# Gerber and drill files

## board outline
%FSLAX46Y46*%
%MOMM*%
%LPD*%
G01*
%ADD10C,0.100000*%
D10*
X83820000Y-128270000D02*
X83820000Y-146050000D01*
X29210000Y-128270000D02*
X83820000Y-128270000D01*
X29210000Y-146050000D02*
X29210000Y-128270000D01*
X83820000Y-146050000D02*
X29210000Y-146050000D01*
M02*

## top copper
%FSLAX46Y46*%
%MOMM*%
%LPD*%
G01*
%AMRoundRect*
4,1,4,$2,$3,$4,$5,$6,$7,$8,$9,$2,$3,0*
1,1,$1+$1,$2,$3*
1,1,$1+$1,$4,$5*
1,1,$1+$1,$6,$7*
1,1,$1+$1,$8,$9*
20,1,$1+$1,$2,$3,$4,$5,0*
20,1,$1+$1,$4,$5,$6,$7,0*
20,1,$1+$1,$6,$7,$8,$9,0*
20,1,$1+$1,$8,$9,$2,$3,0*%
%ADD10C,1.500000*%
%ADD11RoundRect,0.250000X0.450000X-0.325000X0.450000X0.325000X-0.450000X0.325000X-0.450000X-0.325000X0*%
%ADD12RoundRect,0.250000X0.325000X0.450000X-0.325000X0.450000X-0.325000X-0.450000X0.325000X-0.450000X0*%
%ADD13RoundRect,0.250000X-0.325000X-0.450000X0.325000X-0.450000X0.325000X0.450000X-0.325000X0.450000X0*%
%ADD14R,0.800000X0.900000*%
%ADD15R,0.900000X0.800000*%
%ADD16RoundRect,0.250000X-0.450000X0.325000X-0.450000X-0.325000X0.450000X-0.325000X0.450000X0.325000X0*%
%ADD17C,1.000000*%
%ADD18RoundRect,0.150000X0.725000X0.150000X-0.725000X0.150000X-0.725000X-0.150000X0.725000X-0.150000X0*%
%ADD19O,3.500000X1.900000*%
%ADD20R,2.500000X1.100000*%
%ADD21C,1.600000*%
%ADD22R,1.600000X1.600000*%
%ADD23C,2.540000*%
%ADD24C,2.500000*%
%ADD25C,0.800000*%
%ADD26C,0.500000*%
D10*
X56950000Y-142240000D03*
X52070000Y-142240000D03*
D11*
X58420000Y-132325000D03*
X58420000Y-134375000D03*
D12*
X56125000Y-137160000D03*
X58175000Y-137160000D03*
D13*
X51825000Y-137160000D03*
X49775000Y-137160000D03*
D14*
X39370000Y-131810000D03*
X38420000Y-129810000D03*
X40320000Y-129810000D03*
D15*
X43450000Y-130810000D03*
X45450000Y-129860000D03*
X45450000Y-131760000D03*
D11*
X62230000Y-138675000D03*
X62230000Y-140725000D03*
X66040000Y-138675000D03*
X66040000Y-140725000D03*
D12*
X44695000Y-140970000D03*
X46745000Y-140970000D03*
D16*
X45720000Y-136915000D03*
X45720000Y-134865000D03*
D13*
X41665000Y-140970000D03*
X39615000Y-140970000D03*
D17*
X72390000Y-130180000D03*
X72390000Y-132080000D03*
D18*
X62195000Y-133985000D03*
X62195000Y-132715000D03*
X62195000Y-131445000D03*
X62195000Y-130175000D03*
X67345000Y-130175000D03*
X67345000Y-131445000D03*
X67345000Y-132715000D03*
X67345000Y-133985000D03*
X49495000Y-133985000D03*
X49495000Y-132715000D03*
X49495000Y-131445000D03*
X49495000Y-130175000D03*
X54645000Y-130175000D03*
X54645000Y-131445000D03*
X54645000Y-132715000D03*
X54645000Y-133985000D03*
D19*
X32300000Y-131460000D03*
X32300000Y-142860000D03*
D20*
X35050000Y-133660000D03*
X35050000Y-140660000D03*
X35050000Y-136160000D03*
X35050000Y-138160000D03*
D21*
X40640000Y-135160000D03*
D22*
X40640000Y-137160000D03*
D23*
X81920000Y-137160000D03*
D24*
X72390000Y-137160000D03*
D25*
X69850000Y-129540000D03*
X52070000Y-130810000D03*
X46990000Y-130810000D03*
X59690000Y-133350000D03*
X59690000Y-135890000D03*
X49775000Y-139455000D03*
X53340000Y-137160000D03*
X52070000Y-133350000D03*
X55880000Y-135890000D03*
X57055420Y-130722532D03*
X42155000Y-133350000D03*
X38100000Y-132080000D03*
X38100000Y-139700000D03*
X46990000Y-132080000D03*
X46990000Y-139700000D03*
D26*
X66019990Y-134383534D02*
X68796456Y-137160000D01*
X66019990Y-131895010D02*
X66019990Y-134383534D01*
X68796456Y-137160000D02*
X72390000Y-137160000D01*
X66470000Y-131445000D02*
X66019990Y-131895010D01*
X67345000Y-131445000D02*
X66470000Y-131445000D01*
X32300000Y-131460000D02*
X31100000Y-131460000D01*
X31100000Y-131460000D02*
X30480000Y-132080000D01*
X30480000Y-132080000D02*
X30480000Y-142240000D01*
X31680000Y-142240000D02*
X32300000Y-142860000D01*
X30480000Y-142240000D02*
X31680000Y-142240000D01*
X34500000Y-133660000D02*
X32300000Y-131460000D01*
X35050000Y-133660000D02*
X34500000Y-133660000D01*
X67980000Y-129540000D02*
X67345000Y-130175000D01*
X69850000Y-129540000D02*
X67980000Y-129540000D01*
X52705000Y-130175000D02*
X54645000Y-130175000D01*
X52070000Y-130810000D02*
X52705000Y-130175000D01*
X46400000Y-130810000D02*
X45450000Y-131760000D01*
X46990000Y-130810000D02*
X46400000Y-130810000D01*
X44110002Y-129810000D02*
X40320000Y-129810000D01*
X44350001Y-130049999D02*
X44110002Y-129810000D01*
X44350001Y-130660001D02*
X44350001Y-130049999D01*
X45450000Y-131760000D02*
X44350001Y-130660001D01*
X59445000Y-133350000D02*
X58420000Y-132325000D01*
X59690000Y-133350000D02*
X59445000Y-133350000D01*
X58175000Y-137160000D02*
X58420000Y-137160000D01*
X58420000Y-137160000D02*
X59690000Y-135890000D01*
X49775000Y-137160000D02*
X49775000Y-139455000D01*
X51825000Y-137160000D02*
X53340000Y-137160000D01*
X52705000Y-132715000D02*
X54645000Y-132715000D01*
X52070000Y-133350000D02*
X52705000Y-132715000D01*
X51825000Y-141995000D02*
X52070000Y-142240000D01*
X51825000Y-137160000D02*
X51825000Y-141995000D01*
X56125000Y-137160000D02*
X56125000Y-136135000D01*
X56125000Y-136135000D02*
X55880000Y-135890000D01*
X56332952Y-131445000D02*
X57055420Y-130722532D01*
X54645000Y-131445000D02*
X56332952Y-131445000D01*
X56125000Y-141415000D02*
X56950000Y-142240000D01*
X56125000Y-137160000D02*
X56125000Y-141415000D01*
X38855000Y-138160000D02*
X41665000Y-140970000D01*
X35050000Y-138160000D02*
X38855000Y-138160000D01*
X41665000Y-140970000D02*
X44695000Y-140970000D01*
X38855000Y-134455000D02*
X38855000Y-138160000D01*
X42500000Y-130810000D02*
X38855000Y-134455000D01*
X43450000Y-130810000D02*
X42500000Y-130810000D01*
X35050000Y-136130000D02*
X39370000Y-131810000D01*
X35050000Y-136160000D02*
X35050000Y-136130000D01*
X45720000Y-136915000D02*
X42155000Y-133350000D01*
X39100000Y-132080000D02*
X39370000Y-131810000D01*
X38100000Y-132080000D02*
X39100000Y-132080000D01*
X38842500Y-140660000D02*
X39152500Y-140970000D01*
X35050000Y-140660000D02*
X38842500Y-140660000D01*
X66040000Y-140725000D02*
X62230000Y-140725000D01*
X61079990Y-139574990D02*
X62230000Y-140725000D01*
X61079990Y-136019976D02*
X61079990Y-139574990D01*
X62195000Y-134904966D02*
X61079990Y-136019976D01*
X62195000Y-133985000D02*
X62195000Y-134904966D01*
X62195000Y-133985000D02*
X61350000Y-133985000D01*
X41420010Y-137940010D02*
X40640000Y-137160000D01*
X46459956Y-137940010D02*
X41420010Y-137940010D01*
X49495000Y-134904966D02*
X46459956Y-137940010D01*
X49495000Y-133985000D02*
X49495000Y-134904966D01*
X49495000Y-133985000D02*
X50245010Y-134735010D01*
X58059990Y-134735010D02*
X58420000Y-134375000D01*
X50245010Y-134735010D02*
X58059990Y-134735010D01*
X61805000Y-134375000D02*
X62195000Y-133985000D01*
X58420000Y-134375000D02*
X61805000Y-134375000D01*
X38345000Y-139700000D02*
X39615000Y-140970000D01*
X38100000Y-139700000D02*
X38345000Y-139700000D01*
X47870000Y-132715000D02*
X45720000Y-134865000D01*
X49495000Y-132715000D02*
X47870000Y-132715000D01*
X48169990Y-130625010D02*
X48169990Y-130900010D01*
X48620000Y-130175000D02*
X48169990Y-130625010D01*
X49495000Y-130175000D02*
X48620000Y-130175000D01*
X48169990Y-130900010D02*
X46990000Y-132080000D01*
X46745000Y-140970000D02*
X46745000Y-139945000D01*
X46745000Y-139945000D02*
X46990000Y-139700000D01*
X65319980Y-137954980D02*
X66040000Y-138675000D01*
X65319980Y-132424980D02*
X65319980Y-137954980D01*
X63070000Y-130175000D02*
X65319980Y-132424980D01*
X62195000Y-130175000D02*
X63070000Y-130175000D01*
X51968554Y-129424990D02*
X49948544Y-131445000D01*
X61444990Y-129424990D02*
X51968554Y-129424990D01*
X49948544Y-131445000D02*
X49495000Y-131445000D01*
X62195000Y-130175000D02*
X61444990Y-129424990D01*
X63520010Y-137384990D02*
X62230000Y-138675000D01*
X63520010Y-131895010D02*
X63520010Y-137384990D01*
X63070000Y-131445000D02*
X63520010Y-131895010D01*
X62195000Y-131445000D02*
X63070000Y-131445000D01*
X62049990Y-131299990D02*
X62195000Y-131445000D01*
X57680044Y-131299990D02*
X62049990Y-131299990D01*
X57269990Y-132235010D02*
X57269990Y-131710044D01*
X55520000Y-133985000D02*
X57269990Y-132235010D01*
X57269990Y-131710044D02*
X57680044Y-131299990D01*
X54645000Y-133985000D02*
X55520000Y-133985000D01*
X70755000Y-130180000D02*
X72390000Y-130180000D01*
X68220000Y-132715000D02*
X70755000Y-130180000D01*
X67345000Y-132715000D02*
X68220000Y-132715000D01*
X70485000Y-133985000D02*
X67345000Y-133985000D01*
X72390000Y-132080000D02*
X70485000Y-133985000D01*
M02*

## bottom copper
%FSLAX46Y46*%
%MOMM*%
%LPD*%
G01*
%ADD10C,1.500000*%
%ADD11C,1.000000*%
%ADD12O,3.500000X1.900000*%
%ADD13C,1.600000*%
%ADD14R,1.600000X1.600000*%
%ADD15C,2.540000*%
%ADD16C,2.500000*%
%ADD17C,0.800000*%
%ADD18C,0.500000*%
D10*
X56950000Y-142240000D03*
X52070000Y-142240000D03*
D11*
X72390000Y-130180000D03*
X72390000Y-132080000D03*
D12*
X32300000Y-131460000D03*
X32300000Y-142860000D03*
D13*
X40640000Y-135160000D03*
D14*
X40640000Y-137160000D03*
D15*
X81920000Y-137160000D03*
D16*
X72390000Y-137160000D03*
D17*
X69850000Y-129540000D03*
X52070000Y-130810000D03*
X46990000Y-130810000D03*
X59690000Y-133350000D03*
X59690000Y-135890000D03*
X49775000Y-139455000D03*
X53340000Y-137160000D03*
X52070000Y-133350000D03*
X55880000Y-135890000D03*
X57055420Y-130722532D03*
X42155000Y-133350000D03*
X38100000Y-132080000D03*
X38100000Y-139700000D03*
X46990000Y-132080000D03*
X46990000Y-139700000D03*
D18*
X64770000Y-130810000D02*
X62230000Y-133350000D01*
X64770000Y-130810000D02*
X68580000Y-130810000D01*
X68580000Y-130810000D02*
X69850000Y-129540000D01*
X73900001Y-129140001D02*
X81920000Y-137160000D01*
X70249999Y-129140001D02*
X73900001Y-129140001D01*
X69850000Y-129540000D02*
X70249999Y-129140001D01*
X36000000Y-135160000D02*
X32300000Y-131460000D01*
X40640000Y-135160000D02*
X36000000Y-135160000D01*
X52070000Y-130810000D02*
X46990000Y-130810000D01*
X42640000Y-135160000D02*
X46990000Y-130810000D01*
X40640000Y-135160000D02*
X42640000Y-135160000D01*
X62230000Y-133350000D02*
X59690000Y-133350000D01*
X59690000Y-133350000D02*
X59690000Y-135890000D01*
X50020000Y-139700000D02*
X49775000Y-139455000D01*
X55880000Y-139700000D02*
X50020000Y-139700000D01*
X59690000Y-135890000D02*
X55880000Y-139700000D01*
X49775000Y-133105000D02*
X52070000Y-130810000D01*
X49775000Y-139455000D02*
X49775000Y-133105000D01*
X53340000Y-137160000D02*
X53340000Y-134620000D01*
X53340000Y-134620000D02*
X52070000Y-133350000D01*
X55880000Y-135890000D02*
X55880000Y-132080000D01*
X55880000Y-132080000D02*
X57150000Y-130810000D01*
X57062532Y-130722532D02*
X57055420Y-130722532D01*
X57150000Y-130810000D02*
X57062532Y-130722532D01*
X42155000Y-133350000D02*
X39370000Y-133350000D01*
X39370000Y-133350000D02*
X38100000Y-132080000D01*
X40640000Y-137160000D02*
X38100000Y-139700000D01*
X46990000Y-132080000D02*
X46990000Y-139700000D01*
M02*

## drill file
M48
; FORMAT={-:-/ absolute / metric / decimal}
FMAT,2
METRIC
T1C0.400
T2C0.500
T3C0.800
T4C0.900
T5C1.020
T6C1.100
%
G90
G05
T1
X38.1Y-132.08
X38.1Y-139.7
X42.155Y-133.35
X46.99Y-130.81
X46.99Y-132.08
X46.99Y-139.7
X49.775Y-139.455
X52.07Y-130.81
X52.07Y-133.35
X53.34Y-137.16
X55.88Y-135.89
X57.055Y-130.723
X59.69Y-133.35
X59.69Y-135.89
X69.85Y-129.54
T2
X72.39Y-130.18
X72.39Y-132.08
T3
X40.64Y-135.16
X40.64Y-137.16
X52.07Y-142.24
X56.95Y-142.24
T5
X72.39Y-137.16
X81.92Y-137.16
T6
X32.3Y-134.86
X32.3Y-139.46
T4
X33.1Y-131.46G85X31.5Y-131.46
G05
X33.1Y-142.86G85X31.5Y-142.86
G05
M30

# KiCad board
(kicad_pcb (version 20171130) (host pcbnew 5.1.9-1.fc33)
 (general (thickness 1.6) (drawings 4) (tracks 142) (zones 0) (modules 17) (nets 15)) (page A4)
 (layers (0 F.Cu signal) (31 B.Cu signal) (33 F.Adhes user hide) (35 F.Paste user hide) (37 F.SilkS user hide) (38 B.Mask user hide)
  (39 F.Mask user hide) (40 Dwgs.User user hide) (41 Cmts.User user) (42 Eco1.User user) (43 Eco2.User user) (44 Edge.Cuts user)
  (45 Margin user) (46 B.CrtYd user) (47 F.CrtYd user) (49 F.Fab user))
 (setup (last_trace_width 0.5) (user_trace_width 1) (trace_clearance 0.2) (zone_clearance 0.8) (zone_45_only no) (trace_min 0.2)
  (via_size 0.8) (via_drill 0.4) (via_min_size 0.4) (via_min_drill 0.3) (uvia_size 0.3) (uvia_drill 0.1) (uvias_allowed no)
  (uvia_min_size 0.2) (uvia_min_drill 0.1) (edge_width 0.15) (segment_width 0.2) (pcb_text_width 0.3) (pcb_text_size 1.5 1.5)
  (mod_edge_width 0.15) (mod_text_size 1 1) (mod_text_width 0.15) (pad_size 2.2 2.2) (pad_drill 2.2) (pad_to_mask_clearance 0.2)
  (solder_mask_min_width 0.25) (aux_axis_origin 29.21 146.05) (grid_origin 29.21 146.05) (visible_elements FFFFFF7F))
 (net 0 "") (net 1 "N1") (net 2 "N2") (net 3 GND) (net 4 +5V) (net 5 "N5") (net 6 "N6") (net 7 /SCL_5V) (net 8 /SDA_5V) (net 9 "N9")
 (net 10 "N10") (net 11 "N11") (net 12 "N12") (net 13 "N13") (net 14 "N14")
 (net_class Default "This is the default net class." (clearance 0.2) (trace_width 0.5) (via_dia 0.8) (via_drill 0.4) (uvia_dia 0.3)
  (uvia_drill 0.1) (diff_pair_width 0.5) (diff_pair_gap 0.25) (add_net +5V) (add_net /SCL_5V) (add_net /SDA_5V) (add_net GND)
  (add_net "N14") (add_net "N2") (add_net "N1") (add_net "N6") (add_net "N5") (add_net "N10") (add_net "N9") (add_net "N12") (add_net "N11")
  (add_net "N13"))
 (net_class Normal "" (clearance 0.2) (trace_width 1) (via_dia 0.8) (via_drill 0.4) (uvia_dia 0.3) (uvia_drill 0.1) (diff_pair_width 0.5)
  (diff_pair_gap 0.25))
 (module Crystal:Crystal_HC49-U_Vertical (layer F.Cu) (at 52.07 142.24)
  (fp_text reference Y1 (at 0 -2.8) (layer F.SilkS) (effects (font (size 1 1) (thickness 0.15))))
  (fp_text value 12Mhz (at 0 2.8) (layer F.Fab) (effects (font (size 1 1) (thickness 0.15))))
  (pad 2 thru_hole circle (at 4.88 0) (size 1.5 1.5) (drill 0.8) (layers *.Cu *.Mask) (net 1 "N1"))
  (pad 1 thru_hole circle (at 0 0) (size 1.5 1.5) (drill 0.8) (layers *.Cu *.Mask) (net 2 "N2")))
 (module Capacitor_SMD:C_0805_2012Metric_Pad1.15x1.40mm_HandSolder (layer F.Cu) (at 58.42 133.35 90)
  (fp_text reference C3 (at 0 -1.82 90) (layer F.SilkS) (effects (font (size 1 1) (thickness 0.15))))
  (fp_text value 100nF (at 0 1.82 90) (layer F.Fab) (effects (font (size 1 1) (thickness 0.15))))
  (pad 2 smd roundrect (at 1.025 0 90) (size 1.15 1.4) (layers F.Cu F.Paste F.Mask) (roundrect_rratio 0.217391) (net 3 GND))
  (pad 1 smd roundrect (at -1.025 0 90) (size 1.15 1.4) (layers F.Cu F.Paste F.Mask) (roundrect_rratio 0.217391) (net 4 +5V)))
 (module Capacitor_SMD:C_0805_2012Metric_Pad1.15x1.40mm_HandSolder (layer F.Cu) (at 57.15 137.16 180)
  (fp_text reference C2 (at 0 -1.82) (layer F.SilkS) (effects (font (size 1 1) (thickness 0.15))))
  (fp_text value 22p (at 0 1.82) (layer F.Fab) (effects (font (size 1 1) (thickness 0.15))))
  (pad 2 smd roundrect (at 1.025 0 180) (size 1.15 1.4) (layers F.Cu F.Paste F.Mask) (roundrect_rratio 0.217391) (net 1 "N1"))
  (pad 1 smd roundrect (at -1.025 0 180) (size 1.15 1.4) (layers F.Cu F.Paste F.Mask) (roundrect_rratio 0.217391) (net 3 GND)))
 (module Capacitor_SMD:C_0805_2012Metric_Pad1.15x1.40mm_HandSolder (layer F.Cu) (at 50.8 137.16)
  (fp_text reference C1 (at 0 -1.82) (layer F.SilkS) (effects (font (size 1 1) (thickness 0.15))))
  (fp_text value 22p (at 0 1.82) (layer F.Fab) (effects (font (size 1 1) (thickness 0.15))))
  (pad 2 smd roundrect (at 1.025 0) (size 1.15 1.4) (layers F.Cu F.Paste F.Mask) (roundrect_rratio 0.217391) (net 2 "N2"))
  (pad 1 smd roundrect (at -1.025 0) (size 1.15 1.4) (layers F.Cu F.Paste F.Mask) (roundrect_rratio 0.217391) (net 3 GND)))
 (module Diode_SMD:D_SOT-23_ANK (layer F.Cu) (at 39.37 130.81 270)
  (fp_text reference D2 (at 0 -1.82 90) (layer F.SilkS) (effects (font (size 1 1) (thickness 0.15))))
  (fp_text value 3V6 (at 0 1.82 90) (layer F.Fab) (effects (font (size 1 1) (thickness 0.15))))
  (pad 1 smd rect (at 1 0 270) (size 0.9 0.8) (layers F.Cu F.Paste F.Mask) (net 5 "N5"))
  (pad "" smd rect (at -1 0.95 270) (size 0.9 0.8) (layers F.Cu F.Paste F.Mask))
  (pad 2 smd rect (at -1 -0.95 270) (size 0.9 0.8) (layers F.Cu F.Paste F.Mask) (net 3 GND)))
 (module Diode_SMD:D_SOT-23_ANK (layer F.Cu) (at 44.45 130.81 180)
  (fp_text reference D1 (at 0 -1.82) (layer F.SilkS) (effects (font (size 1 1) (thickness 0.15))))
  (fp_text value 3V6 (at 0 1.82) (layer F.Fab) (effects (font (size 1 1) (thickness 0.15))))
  (pad 1 smd rect (at 1 0 180) (size 0.9 0.8) (layers F.Cu F.Paste F.Mask) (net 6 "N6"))
  (pad "" smd rect (at -1 0.95 180) (size 0.9 0.8) (layers F.Cu F.Paste F.Mask))
  (pad 2 smd rect (at -1 -0.95 180) (size 0.9 0.8) (layers F.Cu F.Paste F.Mask) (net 3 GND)))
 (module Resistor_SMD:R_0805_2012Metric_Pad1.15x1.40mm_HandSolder (layer F.Cu) (at 62.23 139.7 90)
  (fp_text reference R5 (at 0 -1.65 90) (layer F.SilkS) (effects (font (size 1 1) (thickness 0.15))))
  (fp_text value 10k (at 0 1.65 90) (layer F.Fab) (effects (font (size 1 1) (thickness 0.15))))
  (pad 2 smd roundrect (at 1.025 0 90) (size 1.15 1.4) (layers F.Cu F.Paste F.Mask) (roundrect_rratio 0.217391) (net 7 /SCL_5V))
  (pad 1 smd roundrect (at -1.025 0 90) (size 1.15 1.4) (layers F.Cu F.Paste F.Mask) (roundrect_rratio 0.217391) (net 4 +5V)))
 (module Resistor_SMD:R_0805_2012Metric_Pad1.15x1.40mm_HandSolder (layer F.Cu) (at 66.04 139.7 90)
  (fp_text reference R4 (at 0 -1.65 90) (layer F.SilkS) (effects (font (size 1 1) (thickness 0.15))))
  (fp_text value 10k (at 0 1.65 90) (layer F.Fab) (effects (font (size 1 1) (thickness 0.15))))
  (pad 2 smd roundrect (at 1.025 0 90) (size 1.15 1.4) (layers F.Cu F.Paste F.Mask) (roundrect_rratio 0.217391) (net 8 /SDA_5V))
  (pad 1 smd roundrect (at -1.025 0 90) (size 1.15 1.4) (layers F.Cu F.Paste F.Mask) (roundrect_rratio 0.217391) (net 4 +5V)))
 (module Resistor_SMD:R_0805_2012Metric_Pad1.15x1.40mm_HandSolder (layer F.Cu) (at 45.72 140.97 180)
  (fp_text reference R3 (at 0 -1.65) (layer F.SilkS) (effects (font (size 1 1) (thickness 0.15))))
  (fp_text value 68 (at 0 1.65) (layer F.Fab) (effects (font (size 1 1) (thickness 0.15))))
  (pad 2 smd roundrect (at 1.025 0 180) (size 1.15 1.4) (layers F.Cu F.Paste F.Mask) (roundrect_rratio 0.217391) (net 6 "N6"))
  (pad 1 smd roundrect (at -1.025 0 180) (size 1.15 1.4) (layers F.Cu F.Paste F.Mask) (roundrect_rratio 0.217391) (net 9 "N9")))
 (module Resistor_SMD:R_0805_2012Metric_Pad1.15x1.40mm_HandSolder (layer F.Cu) (at 45.72 135.89 270)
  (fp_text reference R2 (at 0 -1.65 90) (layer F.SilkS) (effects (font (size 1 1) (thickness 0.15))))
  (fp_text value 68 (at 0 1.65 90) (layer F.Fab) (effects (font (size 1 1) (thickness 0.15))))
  (pad 2 smd roundrect (at 1.025 0 270) (size 1.15 1.4) (layers F.Cu F.Paste F.Mask) (roundrect_rratio 0.217391) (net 5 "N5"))
  (pad 1 smd roundrect (at -1.025 0 270) (size 1.15 1.4) (layers F.Cu F.Paste F.Mask) (roundrect_rratio 0.217391) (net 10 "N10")))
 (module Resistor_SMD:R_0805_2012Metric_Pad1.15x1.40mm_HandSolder (layer F.Cu) (at 40.64 140.97)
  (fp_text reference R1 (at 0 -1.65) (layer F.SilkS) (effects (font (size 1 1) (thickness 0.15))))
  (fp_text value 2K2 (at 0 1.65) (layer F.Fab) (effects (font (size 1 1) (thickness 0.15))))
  (pad 2 smd roundrect (at 1.025 0) (size 1.15 1.4) (layers F.Cu F.Paste F.Mask) (roundrect_rratio 0.217391) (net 6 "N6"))
  (pad 1 smd roundrect (at -1.025 0) (size 1.15 1.4) (layers F.Cu F.Paste F.Mask) (roundrect_rratio 0.217391) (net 4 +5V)))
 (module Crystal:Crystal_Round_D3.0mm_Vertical (layer F.Cu) (at 72.39 132.08 90)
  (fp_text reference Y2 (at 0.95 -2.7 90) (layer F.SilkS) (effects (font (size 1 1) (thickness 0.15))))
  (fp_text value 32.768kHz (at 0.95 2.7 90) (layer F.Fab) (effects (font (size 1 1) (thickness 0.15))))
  (pad 2 thru_hole circle (at 1.9 0 90) (size 1 1) (drill 0.5) (layers *.Cu *.Mask) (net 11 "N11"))
  (pad 1 thru_hole circle (at 0 0 90) (size 1 1) (drill 0.5) (layers *.Cu *.Mask) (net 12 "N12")))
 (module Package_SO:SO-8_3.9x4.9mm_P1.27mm (layer F.Cu) (at 64.77 132.08 180)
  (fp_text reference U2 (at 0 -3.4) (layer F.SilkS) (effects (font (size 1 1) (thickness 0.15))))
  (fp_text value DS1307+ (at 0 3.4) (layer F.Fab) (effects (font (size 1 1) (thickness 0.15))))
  (pad 8 smd roundrect (at 2.575 -1.905 180) (size 1.75 0.6) (layers F.Cu F.Paste F.Mask) (roundrect_rratio 0.25) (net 4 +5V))
  (pad 7 smd roundrect (at 2.575 -0.635 180) (size 1.75 0.6) (layers F.Cu F.Paste F.Mask) (roundrect_rratio 0.25) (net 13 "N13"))
  (pad 6 smd roundrect (at 2.575 0.635 180) (size 1.75 0.6) (layers F.Cu F.Paste F.Mask) (roundrect_rratio 0.25) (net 7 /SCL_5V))
  (pad 5 smd roundrect (at 2.575 1.905 180) (size 1.75 0.6) (layers F.Cu F.Paste F.Mask) (roundrect_rratio 0.25) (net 8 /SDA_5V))
  (pad 4 smd roundrect (at -2.575 1.905 180) (size 1.75 0.6) (layers F.Cu F.Paste F.Mask) (roundrect_rratio 0.25) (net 3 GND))
  (pad 3 smd roundrect (at -2.575 0.635 180) (size 1.75 0.6) (layers F.Cu F.Paste F.Mask) (roundrect_rratio 0.25) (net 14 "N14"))
  (pad 2 smd roundrect (at -2.575 -0.635 180) (size 1.75 0.6) (layers F.Cu F.Paste F.Mask) (roundrect_rratio 0.25) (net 11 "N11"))
  (pad 1 smd roundrect (at -2.575 -1.905 180) (size 1.75 0.6) (layers F.Cu F.Paste F.Mask) (roundrect_rratio 0.25) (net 12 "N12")))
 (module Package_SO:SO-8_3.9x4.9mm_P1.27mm (layer F.Cu) (at 52.07 132.08 180)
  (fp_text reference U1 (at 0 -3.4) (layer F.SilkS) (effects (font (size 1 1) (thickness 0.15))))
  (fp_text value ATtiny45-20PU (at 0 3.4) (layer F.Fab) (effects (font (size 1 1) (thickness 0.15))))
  (pad 8 smd roundrect (at 2.575 -1.905 180) (size 1.75 0.6) (layers F.Cu F.Paste F.Mask) (roundrect_rratio 0.25) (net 4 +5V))
  (pad 7 smd roundrect (at 2.575 -0.635 180) (size 1.75 0.6) (layers F.Cu F.Paste F.Mask) (roundrect_rratio 0.25) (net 10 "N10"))
  (pad 6 smd roundrect (at 2.575 0.635 180) (size 1.75 0.6) (layers F.Cu F.Paste F.Mask) (roundrect_rratio 0.25) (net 8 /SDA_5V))
  (pad 5 smd roundrect (at 2.575 1.905 180) (size 1.75 0.6) (layers F.Cu F.Paste F.Mask) (roundrect_rratio 0.25) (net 9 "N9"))
  (pad 4 smd roundrect (at -2.575 1.905 180) (size 1.75 0.6) (layers F.Cu F.Paste F.Mask) (roundrect_rratio 0.25) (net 3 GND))
  (pad 3 smd roundrect (at -2.575 0.635 180) (size 1.75 0.6) (layers F.Cu F.Paste F.Mask) (roundrect_rratio 0.25) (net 1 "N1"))
  (pad 2 smd roundrect (at -2.575 -0.635 180) (size 1.75 0.6) (layers F.Cu F.Paste F.Mask) (roundrect_rratio 0.25) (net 2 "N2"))
  (pad 1 smd roundrect (at -2.575 -1.905 180) (size 1.75 0.6) (layers F.Cu F.Paste F.Mask) (roundrect_rratio 0.25) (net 7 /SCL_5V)))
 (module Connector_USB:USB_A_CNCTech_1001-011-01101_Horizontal (layer F.Cu) (at 25.4 137.16 180)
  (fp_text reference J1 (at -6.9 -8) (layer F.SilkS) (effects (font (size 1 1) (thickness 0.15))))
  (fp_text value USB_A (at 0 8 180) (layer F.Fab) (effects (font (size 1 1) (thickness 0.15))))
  (pad "" np_thru_hole circle (at -6.9 2.3 180) (size 1.1 1.1) (drill 1.1) (layers *.Cu *.Mask))
  (pad "" np_thru_hole circle (at -6.9 -2.3 180) (size 1.1 1.1) (drill 1.1) (layers *.Cu *.Mask))
  (pad 5 thru_hole oval (at -6.9 5.7 180) (size 3.5 1.9) (drill oval 2.5 0.9) (layers *.Cu *.Mask) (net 3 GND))
  (pad 5 thru_hole oval (at -6.9 -5.7 180) (size 3.5 1.9) (drill oval 2.5 0.9) (layers *.Cu *.Mask) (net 3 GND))
  (pad 4 smd rect (at -9.65 3.5 180) (size 2.5 1.1) (layers F.Cu F.Paste F.Mask) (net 3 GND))
  (pad 1 smd rect (at -9.65 -3.5 180) (size 2.5 1.1) (layers F.Cu F.Paste F.Mask) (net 4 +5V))
  (pad 3 smd rect (at -9.65 1 180) (size 2.5 1.1) (layers F.Cu F.Paste F.Mask) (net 5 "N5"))
  (pad 2 smd rect (at -9.65 -1 180) (size 2.5 1.1) (layers F.Cu F.Paste F.Mask) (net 6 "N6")))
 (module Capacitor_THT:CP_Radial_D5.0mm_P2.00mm (layer F.Cu) (at 40.64 137.16 90)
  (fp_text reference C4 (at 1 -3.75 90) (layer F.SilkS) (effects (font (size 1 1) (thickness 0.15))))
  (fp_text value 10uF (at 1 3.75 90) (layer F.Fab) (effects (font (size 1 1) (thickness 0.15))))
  (pad 2 thru_hole circle (at 2 0 90) (size 1.6 1.6) (drill 0.8) (layers *.Cu *.Mask) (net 3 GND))
  (pad 1 thru_hole rect (at 0 0 90) (size 1.6 1.6) (drill 0.8) (layers *.Cu *.Mask) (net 4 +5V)))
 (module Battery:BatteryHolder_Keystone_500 (layer F.Cu) (at 72.39 137.16)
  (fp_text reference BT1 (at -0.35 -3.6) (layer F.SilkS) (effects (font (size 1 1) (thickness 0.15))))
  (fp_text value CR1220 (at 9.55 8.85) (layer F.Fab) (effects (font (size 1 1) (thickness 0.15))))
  (pad 2 thru_hole circle (at 9.53 0) (size 2.54 2.54) (drill 1.02) (layers *.Cu *.Mask) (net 3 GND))
  (pad 1 thru_hole circle (at 0 0) (size 2.5 2.5) (drill 1.02) (layers *.Cu *.Mask) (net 14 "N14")))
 (gr_line (start 83.82 128.27) (end 83.82 146.05) (layer Edge.Cuts) (width 0.1))
 (gr_line (start 29.21 128.27) (end 83.82 128.27) (layer Edge.Cuts) (width 0.1))
 (gr_line (start 29.21 146.05) (end 29.21 128.27) (layer Edge.Cuts) (width 0.1))
 (gr_line (start 83.82 146.05) (end 29.21 146.05) (layer Edge.Cuts) (width 0.1))
 (segment (start 66.01999 134.383534) (end 68.796456 137.16) (width 0.5) (layer F.Cu) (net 14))
 (segment (start 66.01999 131.89501) (end 66.01999 134.383534) (width 0.5) (layer F.Cu) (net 14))
 (segment (start 68.796456 137.16) (end 72.39 137.16) (width 0.5) (layer F.Cu) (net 14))
 (segment (start 66.47 131.445) (end 66.01999 131.89501) (width 0.5) (layer F.Cu) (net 14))
 (segment (start 67.345 131.445) (end 66.47 131.445) (width 0.5) (layer F.Cu) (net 14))
 (segment (start 32.3 131.46) (end 31.1 131.46) (width 0.5) (layer F.Cu) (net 3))
 (segment (start 31.1 131.46) (end 30.48 132.08) (width 0.5) (layer F.Cu) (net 3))
 (segment (start 30.48 132.08) (end 30.48 142.24) (width 0.5) (layer F.Cu) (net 3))
 (segment (start 31.68 142.24) (end 32.3 142.86) (width 0.5) (layer F.Cu) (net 3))
 (segment (start 30.48 142.24) (end 31.68 142.24) (width 0.5) (layer F.Cu) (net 3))
 (segment (start 34.5 133.66) (end 32.3 131.46) (width 0.5) (layer F.Cu) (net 3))
 (segment (start 35.05 133.66) (end 34.5 133.66) (width 0.5) (layer F.Cu) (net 3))
 (segment (start 64.77 130.81) (end 62.23 133.35) (width 0.5) (layer B.Cu) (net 3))
 (segment (start 64.77 130.81) (end 68.58 130.81) (width 0.5) (layer B.Cu) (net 3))
 (segment (start 68.58 130.81) (end 69.85 129.54) (width 0.5) (layer B.Cu) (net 3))
 (via (at 69.85 129.54) (size 0.8) (drill 0.4) (layers F.Cu B.Cu) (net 3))
 (segment (start 67.98 129.54) (end 67.345 130.175) (width 0.5) (layer F.Cu) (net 3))
 (segment (start 69.85 129.54) (end 67.98 129.54) (width 0.5) (layer F.Cu) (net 3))
 (segment (start 73.900001 129.140001) (end 81.92 137.16) (width 0.5) (layer B.Cu) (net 3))
 (segment (start 70.249999 129.140001) (end 73.900001 129.140001) (width 0.5) (layer B.Cu) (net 3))
 (segment (start 69.85 129.54) (end 70.249999 129.140001) (width 0.5) (layer B.Cu) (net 3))
 (via (at 52.07 130.81) (size 0.8) (drill 0.4) (layers F.Cu B.Cu) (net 3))
 (segment (start 52.705 130.175) (end 54.645 130.175) (width 0.5) (layer F.Cu) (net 3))
 (segment (start 52.07 130.81) (end 52.705 130.175) (width 0.5) (layer F.Cu) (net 3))
 (segment (start 36 135.16) (end 32.3 131.46) (width 0.5) (layer B.Cu) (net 3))
 (segment (start 40.64 135.16) (end 36 135.16) (width 0.5) (layer B.Cu) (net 3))
 (segment (start 52.07 130.81) (end 46.99 130.81) (width 0.5) (layer B.Cu) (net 3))
 (via (at 46.99 130.81) (size 0.8) (drill 0.4) (layers F.Cu B.Cu) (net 3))
 (segment (start 46.4 130.81) (end 45.45 131.76) (width 0.5) (layer F.Cu) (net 3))
 (segment (start 46.99 130.81) (end 46.4 130.81) (width 0.5) (layer F.Cu) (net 3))
 (segment (start 44.110002 129.81) (end 40.32 129.81) (width 0.5) (layer F.Cu) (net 3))
 (segment (start 44.350001 130.049999) (end 44.110002 129.81) (width 0.5) (layer F.Cu) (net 3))
 (segment (start 44.350001 130.660001) (end 44.350001 130.049999) (width 0.5) (layer F.Cu) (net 3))
 (segment (start 45.45 131.76) (end 44.350001 130.660001) (width 0.5) (layer F.Cu) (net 3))
 (segment (start 42.64 135.16) (end 46.99 130.81) (width 0.5) (layer B.Cu) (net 3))
 (segment (start 40.64 135.16) (end 42.64 135.16) (width 0.5) (layer B.Cu) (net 3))
 (via (at 59.69 133.35) (size 0.8) (drill 0.4) (layers F.Cu B.Cu) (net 3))
 (segment (start 62.23 133.35) (end 59.69 133.35) (width 0.5) (layer B.Cu) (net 3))
 (segment (start 59.445 133.35) (end 58.42 132.325) (width 0.5) (layer F.Cu) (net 3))
 (segment (start 59.69 133.35) (end 59.445 133.35) (width 0.5) (layer F.Cu) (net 3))
 (segment (start 59.69 133.35) (end 59.69 135.89) (width 0.5) (layer B.Cu) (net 3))
 (segment (start 58.175 137.16) (end 58.42 137.16) (width 0.5) (layer F.Cu) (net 3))
 (segment (start 58.42 137.16) (end 59.69 135.89) (width 0.5) (layer F.Cu) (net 3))
 (via (at 59.69 135.89) (size 0.8) (drill 0.4) (layers F.Cu B.Cu) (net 3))
 (segment (start 49.775 137.16) (end 49.775 139.455) (width 0.5) (layer F.Cu) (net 3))
 (via (at 49.775 139.455) (size 0.8) (drill 0.4) (layers F.Cu B.Cu) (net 3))
 (segment (start 50.02 139.7) (end 49.775 139.455) (width 0.5) (layer B.Cu) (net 3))
 (segment (start 55.88 139.7) (end 50.02 139.7) (width 0.5) (layer B.Cu) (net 3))
 (segment (start 59.69 135.89) (end 55.88 139.7) (width 0.5) (layer B.Cu) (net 3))
 (segment (start 49.775 133.105) (end 52.07 130.81) (width 0.5) (layer B.Cu) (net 3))
 (segment (start 49.775 139.455) (end 49.775 133.105) (width 0.5) (layer B.Cu) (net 3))
 (segment (start 51.825 137.16) (end 53.34 137.16) (width 0.5) (layer F.Cu) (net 2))
 (via (at 53.34 137.16) (size 0.8) (drill 0.4) (layers F.Cu B.Cu) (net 2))
 (segment (start 53.34 137.16) (end 53.34 134.62) (width 0.5) (layer B.Cu) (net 2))
 (segment (start 53.34 134.62) (end 52.07 133.35) (width 0.5) (layer B.Cu) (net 2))
 (via (at 52.07 133.35) (size 0.8) (drill 0.4) (layers F.Cu B.Cu) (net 2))
 (segment (start 52.705 132.715) (end 54.645 132.715) (width 0.5) (layer F.Cu) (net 2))
 (segment (start 52.07 133.35) (end 52.705 132.715) (width 0.5) (layer F.Cu) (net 2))
 (segment (start 51.825 141.995) (end 52.07 142.24) (width 0.5) (layer F.Cu) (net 2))
 (segment (start 51.825 137.16) (end 51.825 141.995) (width 0.5) (layer F.Cu) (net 2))
 (segment (start 56.125 137.16) (end 56.125 136.135) (width 0.5) (layer F.Cu) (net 1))
 (via (at 55.88 135.89) (size 0.8) (drill 0.4) (layers F.Cu B.Cu) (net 1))
 (segment (start 56.125 136.135) (end 55.88 135.89) (width 0.5) (layer F.Cu) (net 1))
 (segment (start 55.88 135.89) (end 55.88 132.08) (width 0.5) (layer B.Cu) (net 1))
 (segment (start 55.88 132.08) (end 57.15 130.81) (width 0.5) (layer B.Cu) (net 1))
 (via (at 57.05542 130.722532) (size 0.8) (drill 0.4) (layers F.Cu B.Cu) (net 1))
 (segment (start 57.062532 130.722532) (end 57.05542 130.722532) (width 0.5) (layer B.Cu) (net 1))
 (segment (start 57.15 130.81) (end 57.062532 130.722532) (width 0.5) (layer B.Cu) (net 1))
 (segment (start 56.332952 131.445) (end 57.05542 130.722532) (width 0.5) (layer F.Cu) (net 1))
 (segment (start 54.645 131.445) (end 56.332952 131.445) (width 0.5) (layer F.Cu) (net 1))
 (segment (start 56.125 141.415) (end 56.95 142.24) (width 0.5) (layer F.Cu) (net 1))
 (segment (start 56.125 137.16) (end 56.125 141.415) (width 0.5) (layer F.Cu) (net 1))
 (segment (start 38.855 138.16) (end 41.665 140.97) (width 0.5) (layer F.Cu) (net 6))
 (segment (start 35.05 138.16) (end 38.855 138.16) (width 0.5) (layer F.Cu) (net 6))
 (segment (start 41.665 140.97) (end 44.695 140.97) (width 0.5) (layer F.Cu) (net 6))
 (segment (start 38.855 134.455) (end 38.855 138.16) (width 0.5) (layer F.Cu) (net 6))
 (segment (start 42.5 130.81) (end 38.855 134.455) (width 0.5) (layer F.Cu) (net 6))
 (segment (start 43.45 130.81) (end 42.5 130.81) (width 0.5) (layer F.Cu) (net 6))
 (segment (start 35.05 136.13) (end 39.37 131.81) (width 0.5) (layer F.Cu) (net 5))
 (segment (start 35.05 136.16) (end 35.05 136.13) (width 0.5) (layer F.Cu) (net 5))
 (segment (start 45.72 136.915) (end 42.155 133.35) (width 0.5) (layer F.Cu) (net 5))
 (via (at 42.155 133.35) (size 0.8) (drill 0.4) (layers F.Cu B.Cu) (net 5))
 (segment (start 42.155 133.35) (end 39.37 133.35) (width 0.5) (layer B.Cu) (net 5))
 (segment (start 39.37 133.35) (end 38.1 132.08) (width 0.5) (layer B.Cu) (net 5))
 (via (at 38.1 132.08) (size 0.8) (drill 0.4) (layers F.Cu B.Cu) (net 5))
 (segment (start 39.1 132.08) (end 39.37 131.81) (width 0.5) (layer F.Cu) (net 5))
 (segment (start 38.1 132.08) (end 39.1 132.08) (width 0.5) (layer F.Cu) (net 5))
 (segment (start 38.8425 140.66) (end 39.1525 140.97) (width 0.5) (layer F.Cu) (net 4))
 (segment (start 35.05 140.66) (end 38.8425 140.66) (width 0.5) (layer F.Cu) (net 4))
 (segment (start 66.04 140.725) (end 62.23 140.725) (width 0.5) (layer F.Cu) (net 4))
 (segment (start 61.07999 139.57499) (end 62.23 140.725) (width 0.5) (layer F.Cu) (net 4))
 (segment (start 61.07999 136.019976) (end 61.07999 139.57499) (width 0.5) (layer F.Cu) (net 4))
 (segment (start 62.195 134.904966) (end 61.07999 136.019976) (width 0.5) (layer F.Cu) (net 4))
 (segment (start 62.195 133.985) (end 62.195 134.904966) (width 0.5) (layer F.Cu) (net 4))
 (segment (start 62.195 133.985) (end 61.35 133.985) (width 0.5) (layer F.Cu) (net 4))
 (segment (start 41.42001 137.94001) (end 40.64 137.16) (width 0.5) (layer F.Cu) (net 4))
 (segment (start 46.459956 137.94001) (end 41.42001 137.94001) (width 0.5) (layer F.Cu) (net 4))
 (segment (start 49.495 134.904966) (end 46.459956 137.94001) (width 0.5) (layer F.Cu) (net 4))
 (segment (start 49.495 133.985) (end 49.495 134.904966) (width 0.5) (layer F.Cu) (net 4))
 (segment (start 49.495 133.985) (end 50.24501 134.73501) (width 0.5) (layer F.Cu) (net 4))
 (segment (start 58.05999 134.73501) (end 58.42 134.375) (width 0.5) (layer F.Cu) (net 4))
 (segment (start 50.24501 134.73501) (end 58.05999 134.73501) (width 0.5) (layer F.Cu) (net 4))
 (segment (start 61.805 134.375) (end 62.195 133.985) (width 0.5) (layer F.Cu) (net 4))
 (segment (start 58.42 134.375) (end 61.805 134.375) (width 0.5) (layer F.Cu) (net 4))
 (segment (start 40.64 137.16) (end 38.1 139.7) (width 0.5) (layer B.Cu) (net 4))
 (via (at 38.1 139.7) (size 0.8) (drill 0.4) (layers F.Cu B.Cu) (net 4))
 (segment (start 38.345 139.7) (end 39.615 140.97) (width 0.5) (layer F.Cu) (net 4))
 (segment (start 38.1 139.7) (end 38.345 139.7) (width 0.5) (layer F.Cu) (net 4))
 (segment (start 47.87 132.715) (end 45.72 134.865) (width 0.5) (layer F.Cu) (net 10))
 (segment (start 49.495 132.715) (end 47.87 132.715) (width 0.5) (layer F.Cu) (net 10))
 (segment (start 48.16999 130.62501) (end 48.16999 130.90001) (width 0.5) (layer F.Cu) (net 9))
 (segment (start 48.62 130.175) (end 48.16999 130.62501) (width 0.5) (layer F.Cu) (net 9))
 (segment (start 49.495 130.175) (end 48.62 130.175) (width 0.5) (layer F.Cu) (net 9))
 (segment (start 48.16999 130.90001) (end 46.99 132.08) (width 0.5) (layer F.Cu) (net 9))
 (via (at 46.99 132.08) (size 0.8) (drill 0.4) (layers F.Cu B.Cu) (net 9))
 (segment (start 46.99 132.08) (end 46.99 139.7) (width 0.5) (layer B.Cu) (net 9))
 (segment (start 46.745 140.97) (end 46.745 139.945) (width 0.5) (layer F.Cu) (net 9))
 (segment (start 46.745 139.945) (end 46.99 139.7) (width 0.5) (layer F.Cu) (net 9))
 (via (at 46.99 139.7) (size 0.8) (drill 0.4) (layers F.Cu B.Cu) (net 9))
 (segment (start 65.31998 137.95498) (end 66.04 138.675) (width 0.5) (layer F.Cu) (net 8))
 (segment (start 65.31998 132.42498) (end 65.31998 137.95498) (width 0.5) (layer F.Cu) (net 8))
 (segment (start 63.07 130.175) (end 65.31998 132.42498) (width 0.5) (layer F.Cu) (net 8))
 (segment (start 62.195 130.175) (end 63.07 130.175) (width 0.5) (layer F.Cu) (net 8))
 (segment (start 51.968554 129.42499) (end 49.948544 131.445) (width 0.5) (layer F.Cu) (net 8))
 (segment (start 61.44499 129.42499) (end 51.968554 129.42499) (width 0.5) (layer F.Cu) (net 8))
 (segment (start 49.948544 131.445) (end 49.495 131.445) (width 0.5) (layer F.Cu) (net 8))
 (segment (start 62.195 130.175) (end 61.44499 129.42499) (width 0.5) (layer F.Cu) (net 8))
 (segment (start 63.52001 137.38499) (end 62.23 138.675) (width 0.5) (layer F.Cu) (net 7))
 (segment (start 63.52001 131.89501) (end 63.52001 137.38499) (width 0.5) (layer F.Cu) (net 7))
 (segment (start 63.07 131.445) (end 63.52001 131.89501) (width 0.5) (layer F.Cu) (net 7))
 (segment (start 62.195 131.445) (end 63.07 131.445) (width 0.5) (layer F.Cu) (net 7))
 (segment (start 62.04999 131.29999) (end 62.195 131.445) (width 0.5) (layer F.Cu) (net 7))
 (segment (start 57.680044 131.29999) (end 62.04999 131.29999) (width 0.5) (layer F.Cu) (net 7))
 (segment (start 57.26999 132.23501) (end 57.26999 131.710044) (width 0.5) (layer F.Cu) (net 7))
 (segment (start 55.52 133.985) (end 57.26999 132.23501) (width 0.5) (layer F.Cu) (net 7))
 (segment (start 57.26999 131.710044) (end 57.680044 131.29999) (width 0.5) (layer F.Cu) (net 7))
 (segment (start 54.645 133.985) (end 55.52 133.985) (width 0.5) (layer F.Cu) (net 7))
 (segment (start 70.755 130.18) (end 72.39 130.18) (width 0.5) (layer F.Cu) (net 11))
 (segment (start 68.22 132.715) (end 70.755 130.18) (width 0.5) (layer F.Cu) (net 11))
 (segment (start 67.345 132.715) (end 68.22 132.715) (width 0.5) (layer F.Cu) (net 11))
 (segment (start 70.485 133.985) (end 67.345 133.985) (width 0.5) (layer F.Cu) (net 12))
 (segment (start 72.39 132.08) (end 70.485 133.985) (width 0.5) (layer F.Cu) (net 12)))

